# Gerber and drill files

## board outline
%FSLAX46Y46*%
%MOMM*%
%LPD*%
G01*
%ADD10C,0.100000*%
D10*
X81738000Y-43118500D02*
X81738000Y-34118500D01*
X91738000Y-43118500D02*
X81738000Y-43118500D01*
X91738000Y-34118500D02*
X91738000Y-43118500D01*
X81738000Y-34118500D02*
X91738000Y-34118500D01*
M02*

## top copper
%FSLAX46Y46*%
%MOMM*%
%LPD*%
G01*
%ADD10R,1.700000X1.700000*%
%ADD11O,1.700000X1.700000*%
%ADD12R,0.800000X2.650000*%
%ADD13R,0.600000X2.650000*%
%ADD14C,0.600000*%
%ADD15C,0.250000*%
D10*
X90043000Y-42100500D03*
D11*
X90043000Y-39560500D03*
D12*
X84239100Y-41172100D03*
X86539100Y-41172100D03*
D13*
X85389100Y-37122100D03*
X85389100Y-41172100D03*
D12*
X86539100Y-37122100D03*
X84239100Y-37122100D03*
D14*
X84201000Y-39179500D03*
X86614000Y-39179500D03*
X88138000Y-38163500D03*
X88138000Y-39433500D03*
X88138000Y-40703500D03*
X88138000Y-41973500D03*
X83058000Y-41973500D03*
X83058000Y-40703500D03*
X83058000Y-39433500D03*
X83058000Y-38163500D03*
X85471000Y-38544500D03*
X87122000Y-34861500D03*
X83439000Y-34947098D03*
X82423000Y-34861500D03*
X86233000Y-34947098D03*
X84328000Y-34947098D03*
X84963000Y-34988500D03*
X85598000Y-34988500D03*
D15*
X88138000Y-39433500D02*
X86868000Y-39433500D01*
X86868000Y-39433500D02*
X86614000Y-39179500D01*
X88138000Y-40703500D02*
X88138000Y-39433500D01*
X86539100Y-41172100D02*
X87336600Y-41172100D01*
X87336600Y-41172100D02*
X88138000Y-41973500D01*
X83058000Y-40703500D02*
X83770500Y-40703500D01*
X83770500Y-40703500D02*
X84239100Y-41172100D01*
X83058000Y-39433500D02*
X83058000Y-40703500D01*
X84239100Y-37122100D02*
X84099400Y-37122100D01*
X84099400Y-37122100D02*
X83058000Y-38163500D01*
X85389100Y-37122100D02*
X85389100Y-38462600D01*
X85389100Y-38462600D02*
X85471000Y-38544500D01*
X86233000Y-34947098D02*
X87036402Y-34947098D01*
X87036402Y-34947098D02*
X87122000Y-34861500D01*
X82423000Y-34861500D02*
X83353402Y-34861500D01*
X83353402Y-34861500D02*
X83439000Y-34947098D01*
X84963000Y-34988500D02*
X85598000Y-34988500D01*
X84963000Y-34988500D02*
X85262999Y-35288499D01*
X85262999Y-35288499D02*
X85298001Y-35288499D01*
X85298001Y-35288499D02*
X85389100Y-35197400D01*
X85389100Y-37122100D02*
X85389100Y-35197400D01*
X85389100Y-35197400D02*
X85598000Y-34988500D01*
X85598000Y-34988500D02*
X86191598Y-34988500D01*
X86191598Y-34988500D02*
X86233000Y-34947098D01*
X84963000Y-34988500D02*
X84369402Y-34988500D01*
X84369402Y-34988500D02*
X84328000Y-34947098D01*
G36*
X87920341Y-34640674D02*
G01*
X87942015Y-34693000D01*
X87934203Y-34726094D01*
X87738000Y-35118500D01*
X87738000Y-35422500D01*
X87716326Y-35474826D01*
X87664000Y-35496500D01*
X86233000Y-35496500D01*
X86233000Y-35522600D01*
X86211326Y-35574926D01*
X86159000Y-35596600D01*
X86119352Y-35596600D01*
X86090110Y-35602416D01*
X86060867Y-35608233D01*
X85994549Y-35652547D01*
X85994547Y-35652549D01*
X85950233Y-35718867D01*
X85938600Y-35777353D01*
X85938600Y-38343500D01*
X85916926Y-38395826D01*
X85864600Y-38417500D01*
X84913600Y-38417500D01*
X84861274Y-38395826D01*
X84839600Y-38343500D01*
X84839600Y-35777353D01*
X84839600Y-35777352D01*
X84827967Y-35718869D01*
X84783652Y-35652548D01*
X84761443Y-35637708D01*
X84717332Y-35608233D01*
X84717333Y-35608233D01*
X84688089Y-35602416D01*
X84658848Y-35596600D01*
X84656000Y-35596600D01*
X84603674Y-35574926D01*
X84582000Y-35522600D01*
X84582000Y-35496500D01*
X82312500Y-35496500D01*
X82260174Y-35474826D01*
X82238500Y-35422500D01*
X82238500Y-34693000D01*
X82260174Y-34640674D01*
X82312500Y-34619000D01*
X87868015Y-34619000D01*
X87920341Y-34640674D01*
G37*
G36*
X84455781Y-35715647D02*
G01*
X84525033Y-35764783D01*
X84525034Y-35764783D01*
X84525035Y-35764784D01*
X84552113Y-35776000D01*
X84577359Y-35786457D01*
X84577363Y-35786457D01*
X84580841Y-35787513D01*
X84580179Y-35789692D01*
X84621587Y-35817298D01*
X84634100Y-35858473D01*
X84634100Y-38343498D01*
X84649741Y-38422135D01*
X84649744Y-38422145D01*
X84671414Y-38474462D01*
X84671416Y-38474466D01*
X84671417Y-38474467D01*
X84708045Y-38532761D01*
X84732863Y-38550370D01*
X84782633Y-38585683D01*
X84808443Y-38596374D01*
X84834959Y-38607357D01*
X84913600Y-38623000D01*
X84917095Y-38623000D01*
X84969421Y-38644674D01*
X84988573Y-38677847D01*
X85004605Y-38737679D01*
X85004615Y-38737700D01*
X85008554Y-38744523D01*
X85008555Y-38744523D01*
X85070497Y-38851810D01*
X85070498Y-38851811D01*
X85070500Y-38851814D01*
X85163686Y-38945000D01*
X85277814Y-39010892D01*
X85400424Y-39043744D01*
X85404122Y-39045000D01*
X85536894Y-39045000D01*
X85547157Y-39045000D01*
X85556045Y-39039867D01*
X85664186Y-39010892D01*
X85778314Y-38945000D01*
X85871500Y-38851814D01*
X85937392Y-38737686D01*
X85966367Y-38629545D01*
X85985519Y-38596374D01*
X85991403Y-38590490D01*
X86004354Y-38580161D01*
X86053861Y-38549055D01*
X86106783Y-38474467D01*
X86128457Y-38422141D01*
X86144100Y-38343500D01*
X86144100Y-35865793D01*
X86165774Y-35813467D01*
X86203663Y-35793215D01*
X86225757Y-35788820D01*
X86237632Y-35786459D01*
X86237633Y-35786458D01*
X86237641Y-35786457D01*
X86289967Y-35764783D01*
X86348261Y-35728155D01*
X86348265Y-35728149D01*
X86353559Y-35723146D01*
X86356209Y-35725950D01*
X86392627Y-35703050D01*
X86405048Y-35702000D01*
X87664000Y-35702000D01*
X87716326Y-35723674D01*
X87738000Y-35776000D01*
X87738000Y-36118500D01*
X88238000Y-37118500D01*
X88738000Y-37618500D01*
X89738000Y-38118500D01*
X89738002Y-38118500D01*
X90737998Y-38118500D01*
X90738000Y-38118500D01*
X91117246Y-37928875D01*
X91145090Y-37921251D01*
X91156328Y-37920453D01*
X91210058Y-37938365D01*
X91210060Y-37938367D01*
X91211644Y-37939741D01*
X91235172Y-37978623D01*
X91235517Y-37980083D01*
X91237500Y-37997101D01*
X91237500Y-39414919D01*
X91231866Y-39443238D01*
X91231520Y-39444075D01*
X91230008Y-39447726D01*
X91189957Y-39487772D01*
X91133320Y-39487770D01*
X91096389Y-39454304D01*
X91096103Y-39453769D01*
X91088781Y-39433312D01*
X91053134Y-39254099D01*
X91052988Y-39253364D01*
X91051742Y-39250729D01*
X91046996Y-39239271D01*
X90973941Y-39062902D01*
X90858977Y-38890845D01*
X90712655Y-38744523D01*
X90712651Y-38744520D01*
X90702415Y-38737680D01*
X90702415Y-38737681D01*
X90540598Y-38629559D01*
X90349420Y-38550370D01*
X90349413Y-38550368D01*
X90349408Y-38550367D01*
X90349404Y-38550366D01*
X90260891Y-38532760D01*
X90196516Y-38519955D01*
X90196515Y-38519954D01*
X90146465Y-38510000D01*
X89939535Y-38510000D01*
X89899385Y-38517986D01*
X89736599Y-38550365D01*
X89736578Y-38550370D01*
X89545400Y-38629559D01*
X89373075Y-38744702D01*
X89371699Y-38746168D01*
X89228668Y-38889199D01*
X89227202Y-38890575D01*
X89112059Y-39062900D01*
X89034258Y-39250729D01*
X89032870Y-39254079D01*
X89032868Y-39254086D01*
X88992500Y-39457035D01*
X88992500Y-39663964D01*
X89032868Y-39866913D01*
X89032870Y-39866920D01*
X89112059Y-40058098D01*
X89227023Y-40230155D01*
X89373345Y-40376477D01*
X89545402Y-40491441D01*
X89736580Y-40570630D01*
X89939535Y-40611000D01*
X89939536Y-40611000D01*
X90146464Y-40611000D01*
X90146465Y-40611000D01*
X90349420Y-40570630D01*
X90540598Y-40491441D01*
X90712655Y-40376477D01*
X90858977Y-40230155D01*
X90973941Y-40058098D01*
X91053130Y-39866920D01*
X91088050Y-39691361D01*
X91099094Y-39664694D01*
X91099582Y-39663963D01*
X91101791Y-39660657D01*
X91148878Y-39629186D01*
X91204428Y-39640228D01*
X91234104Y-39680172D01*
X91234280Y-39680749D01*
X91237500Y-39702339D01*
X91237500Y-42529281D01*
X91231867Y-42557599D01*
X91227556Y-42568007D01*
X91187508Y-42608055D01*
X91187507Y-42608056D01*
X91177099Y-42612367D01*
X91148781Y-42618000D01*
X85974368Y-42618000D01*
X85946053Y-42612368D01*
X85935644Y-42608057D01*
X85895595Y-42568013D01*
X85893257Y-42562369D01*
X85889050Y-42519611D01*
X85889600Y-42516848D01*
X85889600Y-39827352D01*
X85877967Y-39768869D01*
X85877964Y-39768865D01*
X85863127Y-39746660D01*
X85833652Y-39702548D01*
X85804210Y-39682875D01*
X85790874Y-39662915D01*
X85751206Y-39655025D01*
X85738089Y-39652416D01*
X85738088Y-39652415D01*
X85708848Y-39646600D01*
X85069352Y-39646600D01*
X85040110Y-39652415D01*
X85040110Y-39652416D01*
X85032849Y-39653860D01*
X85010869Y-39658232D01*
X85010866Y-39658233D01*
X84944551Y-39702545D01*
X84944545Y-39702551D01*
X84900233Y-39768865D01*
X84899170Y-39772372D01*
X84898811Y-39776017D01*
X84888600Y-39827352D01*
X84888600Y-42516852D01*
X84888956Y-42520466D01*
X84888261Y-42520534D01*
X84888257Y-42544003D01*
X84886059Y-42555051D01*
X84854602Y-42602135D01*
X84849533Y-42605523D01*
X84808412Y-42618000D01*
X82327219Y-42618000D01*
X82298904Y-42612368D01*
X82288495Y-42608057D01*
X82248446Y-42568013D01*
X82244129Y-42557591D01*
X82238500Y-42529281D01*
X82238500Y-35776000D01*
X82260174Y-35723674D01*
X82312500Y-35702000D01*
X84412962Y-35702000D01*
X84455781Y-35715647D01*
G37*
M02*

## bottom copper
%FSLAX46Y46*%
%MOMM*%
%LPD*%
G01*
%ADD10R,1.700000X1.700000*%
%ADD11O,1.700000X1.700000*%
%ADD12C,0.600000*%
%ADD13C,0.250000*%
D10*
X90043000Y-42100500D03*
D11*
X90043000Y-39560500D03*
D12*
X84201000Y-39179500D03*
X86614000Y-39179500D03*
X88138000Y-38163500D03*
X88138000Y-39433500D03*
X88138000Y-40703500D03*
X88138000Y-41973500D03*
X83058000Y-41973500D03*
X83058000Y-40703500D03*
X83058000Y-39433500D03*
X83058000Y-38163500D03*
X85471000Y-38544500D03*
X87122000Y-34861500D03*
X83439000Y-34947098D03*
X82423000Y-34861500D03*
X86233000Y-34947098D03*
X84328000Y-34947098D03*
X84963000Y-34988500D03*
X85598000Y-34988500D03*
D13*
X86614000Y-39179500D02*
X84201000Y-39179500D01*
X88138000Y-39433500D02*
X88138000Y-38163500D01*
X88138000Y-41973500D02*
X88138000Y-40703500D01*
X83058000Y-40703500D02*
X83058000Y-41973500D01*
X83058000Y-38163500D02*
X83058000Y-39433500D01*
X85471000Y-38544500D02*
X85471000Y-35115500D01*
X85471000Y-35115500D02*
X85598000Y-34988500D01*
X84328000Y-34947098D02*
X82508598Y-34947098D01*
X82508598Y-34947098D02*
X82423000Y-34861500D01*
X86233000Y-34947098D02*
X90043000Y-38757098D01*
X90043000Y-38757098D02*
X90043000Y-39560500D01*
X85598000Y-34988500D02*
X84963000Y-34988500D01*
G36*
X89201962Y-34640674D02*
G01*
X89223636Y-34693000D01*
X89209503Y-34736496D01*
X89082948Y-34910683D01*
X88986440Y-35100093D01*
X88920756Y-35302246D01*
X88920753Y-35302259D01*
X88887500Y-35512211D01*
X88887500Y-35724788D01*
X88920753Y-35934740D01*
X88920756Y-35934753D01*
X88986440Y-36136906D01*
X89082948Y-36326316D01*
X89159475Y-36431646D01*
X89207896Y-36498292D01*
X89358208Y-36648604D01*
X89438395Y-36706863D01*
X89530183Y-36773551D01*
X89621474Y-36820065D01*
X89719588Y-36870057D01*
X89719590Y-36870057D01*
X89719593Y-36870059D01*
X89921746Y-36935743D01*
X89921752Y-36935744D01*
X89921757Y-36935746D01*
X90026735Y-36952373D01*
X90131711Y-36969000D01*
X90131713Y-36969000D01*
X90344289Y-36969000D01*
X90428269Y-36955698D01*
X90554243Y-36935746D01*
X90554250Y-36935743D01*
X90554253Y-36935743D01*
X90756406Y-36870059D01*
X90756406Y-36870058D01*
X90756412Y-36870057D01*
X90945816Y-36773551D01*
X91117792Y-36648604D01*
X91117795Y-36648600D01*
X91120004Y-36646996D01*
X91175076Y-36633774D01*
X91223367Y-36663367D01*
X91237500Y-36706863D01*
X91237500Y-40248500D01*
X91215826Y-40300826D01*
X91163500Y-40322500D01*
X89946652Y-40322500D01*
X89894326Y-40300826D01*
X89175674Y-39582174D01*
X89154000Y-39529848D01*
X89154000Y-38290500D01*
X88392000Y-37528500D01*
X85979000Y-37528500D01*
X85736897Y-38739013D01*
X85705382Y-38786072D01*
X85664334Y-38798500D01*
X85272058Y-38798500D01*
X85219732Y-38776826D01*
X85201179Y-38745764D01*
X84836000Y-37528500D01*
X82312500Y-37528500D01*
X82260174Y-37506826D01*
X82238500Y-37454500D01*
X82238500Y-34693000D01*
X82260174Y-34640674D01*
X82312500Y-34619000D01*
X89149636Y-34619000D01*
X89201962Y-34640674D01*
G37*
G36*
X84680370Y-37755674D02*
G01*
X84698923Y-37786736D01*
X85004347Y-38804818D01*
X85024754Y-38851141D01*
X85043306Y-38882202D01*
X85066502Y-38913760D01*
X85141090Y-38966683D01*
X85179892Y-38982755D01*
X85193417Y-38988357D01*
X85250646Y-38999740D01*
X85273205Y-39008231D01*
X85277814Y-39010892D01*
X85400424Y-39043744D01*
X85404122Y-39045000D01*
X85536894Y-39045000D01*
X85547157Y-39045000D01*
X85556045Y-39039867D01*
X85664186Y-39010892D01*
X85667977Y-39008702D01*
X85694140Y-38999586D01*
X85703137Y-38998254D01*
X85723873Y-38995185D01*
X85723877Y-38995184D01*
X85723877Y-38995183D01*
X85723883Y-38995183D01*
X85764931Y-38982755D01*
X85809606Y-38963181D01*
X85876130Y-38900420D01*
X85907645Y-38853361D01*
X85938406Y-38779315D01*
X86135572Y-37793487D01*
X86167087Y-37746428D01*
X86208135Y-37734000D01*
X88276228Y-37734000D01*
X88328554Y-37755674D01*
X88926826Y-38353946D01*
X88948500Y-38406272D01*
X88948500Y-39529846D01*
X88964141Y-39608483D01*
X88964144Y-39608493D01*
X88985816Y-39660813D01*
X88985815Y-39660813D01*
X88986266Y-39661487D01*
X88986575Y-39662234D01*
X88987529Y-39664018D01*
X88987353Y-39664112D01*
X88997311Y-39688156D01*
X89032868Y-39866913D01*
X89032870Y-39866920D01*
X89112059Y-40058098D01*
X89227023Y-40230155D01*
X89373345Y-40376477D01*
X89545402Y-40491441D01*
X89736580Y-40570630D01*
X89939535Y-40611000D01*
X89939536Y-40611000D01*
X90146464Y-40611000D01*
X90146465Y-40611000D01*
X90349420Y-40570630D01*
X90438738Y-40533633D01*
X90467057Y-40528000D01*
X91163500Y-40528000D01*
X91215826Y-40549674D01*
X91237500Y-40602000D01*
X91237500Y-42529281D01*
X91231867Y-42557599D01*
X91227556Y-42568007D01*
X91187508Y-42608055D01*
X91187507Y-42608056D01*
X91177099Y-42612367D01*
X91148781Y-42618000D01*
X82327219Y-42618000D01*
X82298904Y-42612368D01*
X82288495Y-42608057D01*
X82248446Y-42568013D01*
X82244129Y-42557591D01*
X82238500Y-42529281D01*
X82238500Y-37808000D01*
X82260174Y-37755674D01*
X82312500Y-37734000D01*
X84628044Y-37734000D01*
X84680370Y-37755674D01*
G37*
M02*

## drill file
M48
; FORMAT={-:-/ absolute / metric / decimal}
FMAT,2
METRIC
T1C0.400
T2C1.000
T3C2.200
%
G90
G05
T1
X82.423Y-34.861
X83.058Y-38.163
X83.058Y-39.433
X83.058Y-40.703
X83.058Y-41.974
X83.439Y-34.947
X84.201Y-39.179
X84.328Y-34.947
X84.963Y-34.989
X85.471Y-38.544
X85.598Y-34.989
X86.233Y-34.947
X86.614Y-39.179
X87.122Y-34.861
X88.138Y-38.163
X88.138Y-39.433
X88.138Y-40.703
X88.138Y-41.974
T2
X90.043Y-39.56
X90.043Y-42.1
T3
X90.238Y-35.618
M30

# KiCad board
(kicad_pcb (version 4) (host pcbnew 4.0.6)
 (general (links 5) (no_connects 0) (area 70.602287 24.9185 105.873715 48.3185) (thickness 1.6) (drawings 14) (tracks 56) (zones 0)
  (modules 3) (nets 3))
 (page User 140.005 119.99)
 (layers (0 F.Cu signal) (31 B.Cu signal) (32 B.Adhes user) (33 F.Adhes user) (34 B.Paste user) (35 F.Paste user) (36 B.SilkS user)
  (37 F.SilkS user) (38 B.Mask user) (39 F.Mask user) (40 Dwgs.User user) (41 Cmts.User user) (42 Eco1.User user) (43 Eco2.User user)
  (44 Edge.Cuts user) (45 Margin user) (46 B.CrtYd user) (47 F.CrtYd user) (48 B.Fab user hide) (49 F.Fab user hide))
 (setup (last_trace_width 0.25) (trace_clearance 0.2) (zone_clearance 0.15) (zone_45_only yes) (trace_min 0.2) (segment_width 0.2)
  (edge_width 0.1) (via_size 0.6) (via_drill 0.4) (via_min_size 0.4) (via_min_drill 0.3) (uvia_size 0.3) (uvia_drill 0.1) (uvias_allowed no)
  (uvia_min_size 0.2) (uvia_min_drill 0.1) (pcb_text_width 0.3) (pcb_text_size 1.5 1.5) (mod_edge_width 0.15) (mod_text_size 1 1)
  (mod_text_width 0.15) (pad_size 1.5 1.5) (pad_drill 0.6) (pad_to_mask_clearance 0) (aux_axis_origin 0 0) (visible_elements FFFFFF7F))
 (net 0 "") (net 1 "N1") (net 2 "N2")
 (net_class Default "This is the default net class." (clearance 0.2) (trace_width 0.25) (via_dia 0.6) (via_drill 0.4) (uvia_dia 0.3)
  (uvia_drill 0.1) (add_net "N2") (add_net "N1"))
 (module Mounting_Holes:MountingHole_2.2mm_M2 (layer F.Cu) (at 90.238 35.6185)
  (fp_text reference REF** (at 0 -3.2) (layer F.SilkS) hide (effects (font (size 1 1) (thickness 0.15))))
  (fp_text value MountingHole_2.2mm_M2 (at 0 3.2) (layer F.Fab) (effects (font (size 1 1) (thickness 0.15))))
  (pad 1 np_thru_hole circle (at 0 0) (size 2.2 2.2) (drill 2.2) (layers *.Cu *.Mask)))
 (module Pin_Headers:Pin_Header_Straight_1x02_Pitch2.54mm (layer F.Cu) (at 90.043 42.1005 180)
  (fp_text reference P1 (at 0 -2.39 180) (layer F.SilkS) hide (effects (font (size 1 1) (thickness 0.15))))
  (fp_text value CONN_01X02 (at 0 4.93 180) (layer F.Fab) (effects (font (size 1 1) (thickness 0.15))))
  (pad 1 thru_hole rect (at 0 0 180) (size 1.7 1.7) (drill 1) (layers *.Cu *.Mask) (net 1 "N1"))
  (pad 2 thru_hole oval (at 0 2.54 180) (size 1.7 1.7) (drill 1) (layers *.Cu *.Mask) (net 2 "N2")))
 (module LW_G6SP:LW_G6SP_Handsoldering (layer F.Cu) (at 84.2391 37.1221)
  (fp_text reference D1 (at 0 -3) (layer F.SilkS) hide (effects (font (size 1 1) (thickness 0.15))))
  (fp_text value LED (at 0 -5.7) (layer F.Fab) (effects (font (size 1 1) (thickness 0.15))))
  (pad 2 smd rect (at 0 4.05) (size 0.8 2.65) (layers F.Cu F.Mask) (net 1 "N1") (solder_mask_margin 0.1))
  (pad 2 smd rect (at 2.3 4.05) (size 0.8 2.65) (layers F.Cu F.Mask) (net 1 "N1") (solder_mask_margin 0.1))
  (pad 1 smd rect (at 1.15 0) (size 0.6 2.65) (layers F.Cu F.Mask) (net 2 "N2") (solder_mask_margin 0.1))
  (pad ~ smd rect (at 1.15 4.05) (size 0.6 2.65) (layers F.Cu F.Mask) (solder_mask_margin 0.1))
  (pad 2 smd rect (at 2.3 0) (size 0.8 2.65) (layers F.Cu F.Mask) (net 1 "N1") (solder_mask_margin 0.1))
  (pad 2 smd rect (at 0 0) (size 0.8 2.65) (layers F.Cu F.Mask) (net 1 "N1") (solder_mask_margin 0.1)))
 (gr_line (start 81.738 43.1185) (end 81.738 34.1185) (layer Edge.Cuts) (width 0.1))
 (gr_line (start 91.738 43.1185) (end 81.738 43.1185) (layer Edge.Cuts) (width 0.1))
 (gr_line (start 91.738 34.1185) (end 91.738 43.1185) (layer Edge.Cuts) (width 0.1))
 (gr_line (start 81.738 34.1185) (end 91.738 34.1185) (layer Edge.Cuts) (width 0.1))
 (segment (start 86.614 39.1795) (end 84.201 39.1795) (width 0.25) (layer B.Cu) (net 1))
 (via (at 84.201 39.1795) (size 0.6) (drill 0.4) (layers F.Cu B.Cu) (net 1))
 (segment (start 88.138 39.4335) (end 86.868 39.4335) (width 0.25) (layer F.Cu) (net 1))
 (segment (start 86.868 39.4335) (end 86.614 39.1795) (width 0.25) (layer F.Cu) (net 1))
 (via (at 86.614 39.1795) (size 0.6) (drill 0.4) (layers F.Cu B.Cu) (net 1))
 (segment (start 88.138 39.4335) (end 88.138 38.1635) (width 0.25) (layer B.Cu) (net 1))
 (via (at 88.138 38.1635) (size 0.6) (drill 0.4) (layers F.Cu B.Cu) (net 1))
 (segment (start 88.138 40.7035) (end 88.138 39.4335) (width 0.25) (layer F.Cu) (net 1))
 (via (at 88.138 39.4335) (size 0.6) (drill 0.4) (layers F.Cu B.Cu) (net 1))
 (segment (start 88.138 41.9735) (end 88.138 40.7035) (width 0.25) (layer B.Cu) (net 1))
 (via (at 88.138 40.7035) (size 0.6) (drill 0.4) (layers F.Cu B.Cu) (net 1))
 (segment (start 86.5391 41.1721) (end 87.3366 41.1721) (width 0.25) (layer F.Cu) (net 1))
 (segment (start 87.3366 41.1721) (end 88.138 41.9735) (width 0.25) (layer F.Cu) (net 1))
 (via (at 88.138 41.9735) (size 0.6) (drill 0.4) (layers F.Cu B.Cu) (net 1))
 (segment (start 83.058 40.7035) (end 83.7705 40.7035) (width 0.25) (layer F.Cu) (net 1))
 (segment (start 83.7705 40.7035) (end 84.2391 41.1721) (width 0.25) (layer F.Cu) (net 1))
 (segment (start 83.058 40.7035) (end 83.058 41.9735) (width 0.25) (layer B.Cu) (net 1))
 (via (at 83.058 41.9735) (size 0.6) (drill 0.4) (layers F.Cu B.Cu) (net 1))
 (segment (start 83.058 39.4335) (end 83.058 40.7035) (width 0.25) (layer F.Cu) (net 1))
 (via (at 83.058 40.7035) (size 0.6) (drill 0.4) (layers F.Cu B.Cu) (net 1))
 (segment (start 83.058 38.1635) (end 83.058 39.4335) (width 0.25) (layer B.Cu) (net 1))
 (via (at 83.058 39.4335) (size 0.6) (drill 0.4) (layers F.Cu B.Cu) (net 1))
 (segment (start 84.2391 37.1221) (end 84.0994 37.1221) (width 0.25) (layer F.Cu) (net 1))
 (via (at 83.058 38.1635) (size 0.6) (drill 0.4) (layers F.Cu B.Cu) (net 1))
 (segment (start 84.0994 37.1221) (end 83.058 38.1635) (width 0.25) (layer F.Cu) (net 1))
 (segment (start 85.471 38.5445) (end 85.471 35.1155) (width 0.25) (layer B.Cu) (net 2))
 (segment (start 85.471 35.1155) (end 85.598 34.9885) (width 0.25) (layer B.Cu) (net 2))
 (segment (start 85.3891 37.1221) (end 85.3891 38.4626) (width 0.25) (layer F.Cu) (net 2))
 (via (at 85.471 38.5445) (size 0.6) (drill 0.4) (layers F.Cu B.Cu) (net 2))
 (segment (start 85.3891 38.4626) (end 85.471 38.5445) (width 0.25) (layer F.Cu) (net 2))
 (segment (start 86.233 34.947098) (end 87.036402 34.947098) (width 0.25) (layer F.Cu) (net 2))
 (segment (start 87.036402 34.947098) (end 87.122 34.8615) (width 0.25) (layer F.Cu) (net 2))
 (via (at 87.122 34.8615) (size 0.6) (drill 0.4) (layers F.Cu B.Cu) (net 2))
 (segment (start 82.423 34.8615) (end 83.353402 34.8615) (width 0.25) (layer F.Cu) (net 2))
 (segment (start 83.353402 34.8615) (end 83.439 34.947098) (width 0.25) (layer F.Cu) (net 2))
 (via (at 83.439 34.947098) (size 0.6) (drill 0.4) (layers F.Cu B.Cu) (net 2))
 (segment (start 84.328 34.947098) (end 82.508598 34.947098) (width 0.25) (layer B.Cu) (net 2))
 (segment (start 82.508598 34.947098) (end 82.423 34.8615) (width 0.25) (layer B.Cu) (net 2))
 (via (at 82.423 34.8615) (size 0.6) (drill 0.4) (layers F.Cu B.Cu) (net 2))
 (segment (start 86.233 34.947098) (end 90.043 38.757098) (width 0.25) (layer B.Cu) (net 2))
 (segment (start 90.043 38.757098) (end 90.043 39.5605) (width 0.25) (layer B.Cu) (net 2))
 (segment (start 84.963 34.9885) (end 85.598 34.9885) (width 0.25) (layer F.Cu) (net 2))
 (segment (start 84.963 34.9885) (end 85.262999 35.288499) (width 0.25) (layer F.Cu) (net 2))
 (segment (start 85.262999 35.288499) (end 85.298001 35.288499) (width 0.25) (layer F.Cu) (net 2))
 (segment (start 85.298001 35.288499) (end 85.3891 35.1974) (width 0.25) (layer F.Cu) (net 2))
 (segment (start 85.3891 37.1221) (end 85.3891 35.1974) (width 0.25) (layer F.Cu) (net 2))
 (segment (start 85.3891 35.1974) (end 85.598 34.9885) (width 0.25) (layer F.Cu) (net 2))
 (segment (start 85.598 34.9885) (end 86.191598 34.9885) (width 0.25) (layer F.Cu) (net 2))
 (segment (start 86.191598 34.9885) (end 86.233 34.947098) (width 0.25) (layer F.Cu) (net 2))
 (via (at 86.233 34.947098) (size 0.6) (drill 0.4) (layers F.Cu B.Cu) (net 2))
 (segment (start 84.963 34.9885) (end 84.369402 34.9885) (width 0.25) (layer F.Cu) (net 2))
 (segment (start 84.369402 34.9885) (end 84.328 34.947098) (width 0.25) (layer F.Cu) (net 2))
 (via (at 84.328 34.947098) (size 0.6) (drill 0.4) (layers F.Cu B.Cu) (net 2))
 (segment (start 85.598 34.9885) (end 84.963 34.9885) (width 0.25) (layer B.Cu) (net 2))
 (via (at 84.963 34.9885) (size 0.6) (drill 0.4) (layers F.Cu B.Cu) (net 2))
 (via (at 85.598 34.9885) (size 0.6) (drill 0.4) (layers F.Cu B.Cu) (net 2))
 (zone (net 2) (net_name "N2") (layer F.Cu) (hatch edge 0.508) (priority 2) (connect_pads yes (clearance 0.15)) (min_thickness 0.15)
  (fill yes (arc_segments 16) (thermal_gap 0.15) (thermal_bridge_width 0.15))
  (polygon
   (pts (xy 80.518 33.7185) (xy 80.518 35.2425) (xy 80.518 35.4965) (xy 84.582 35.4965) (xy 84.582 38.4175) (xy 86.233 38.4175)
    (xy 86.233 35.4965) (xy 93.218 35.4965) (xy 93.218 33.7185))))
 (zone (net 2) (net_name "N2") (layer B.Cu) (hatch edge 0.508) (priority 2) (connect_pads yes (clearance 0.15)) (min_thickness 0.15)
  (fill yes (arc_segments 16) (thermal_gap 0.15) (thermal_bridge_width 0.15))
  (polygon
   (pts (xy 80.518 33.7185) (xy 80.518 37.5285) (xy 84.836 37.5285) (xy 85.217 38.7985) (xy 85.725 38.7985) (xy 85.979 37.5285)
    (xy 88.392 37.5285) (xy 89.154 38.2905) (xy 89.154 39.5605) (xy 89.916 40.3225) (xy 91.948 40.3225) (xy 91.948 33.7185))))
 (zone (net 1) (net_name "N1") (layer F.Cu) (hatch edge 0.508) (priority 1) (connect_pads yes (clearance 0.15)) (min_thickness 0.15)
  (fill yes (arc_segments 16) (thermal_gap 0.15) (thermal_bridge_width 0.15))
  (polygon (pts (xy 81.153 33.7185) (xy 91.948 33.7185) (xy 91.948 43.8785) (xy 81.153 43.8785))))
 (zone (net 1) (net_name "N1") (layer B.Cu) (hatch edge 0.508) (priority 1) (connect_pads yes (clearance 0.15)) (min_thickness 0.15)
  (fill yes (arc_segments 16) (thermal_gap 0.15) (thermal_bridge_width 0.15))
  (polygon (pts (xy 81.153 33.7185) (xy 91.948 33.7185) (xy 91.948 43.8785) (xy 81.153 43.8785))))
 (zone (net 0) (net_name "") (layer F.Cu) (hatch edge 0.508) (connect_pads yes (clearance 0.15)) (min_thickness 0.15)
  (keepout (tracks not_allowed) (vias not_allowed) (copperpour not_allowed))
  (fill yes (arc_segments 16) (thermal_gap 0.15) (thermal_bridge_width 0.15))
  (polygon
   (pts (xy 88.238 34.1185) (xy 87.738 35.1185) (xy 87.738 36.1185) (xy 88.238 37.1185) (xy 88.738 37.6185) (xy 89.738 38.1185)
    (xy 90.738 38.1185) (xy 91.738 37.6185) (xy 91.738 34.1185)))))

